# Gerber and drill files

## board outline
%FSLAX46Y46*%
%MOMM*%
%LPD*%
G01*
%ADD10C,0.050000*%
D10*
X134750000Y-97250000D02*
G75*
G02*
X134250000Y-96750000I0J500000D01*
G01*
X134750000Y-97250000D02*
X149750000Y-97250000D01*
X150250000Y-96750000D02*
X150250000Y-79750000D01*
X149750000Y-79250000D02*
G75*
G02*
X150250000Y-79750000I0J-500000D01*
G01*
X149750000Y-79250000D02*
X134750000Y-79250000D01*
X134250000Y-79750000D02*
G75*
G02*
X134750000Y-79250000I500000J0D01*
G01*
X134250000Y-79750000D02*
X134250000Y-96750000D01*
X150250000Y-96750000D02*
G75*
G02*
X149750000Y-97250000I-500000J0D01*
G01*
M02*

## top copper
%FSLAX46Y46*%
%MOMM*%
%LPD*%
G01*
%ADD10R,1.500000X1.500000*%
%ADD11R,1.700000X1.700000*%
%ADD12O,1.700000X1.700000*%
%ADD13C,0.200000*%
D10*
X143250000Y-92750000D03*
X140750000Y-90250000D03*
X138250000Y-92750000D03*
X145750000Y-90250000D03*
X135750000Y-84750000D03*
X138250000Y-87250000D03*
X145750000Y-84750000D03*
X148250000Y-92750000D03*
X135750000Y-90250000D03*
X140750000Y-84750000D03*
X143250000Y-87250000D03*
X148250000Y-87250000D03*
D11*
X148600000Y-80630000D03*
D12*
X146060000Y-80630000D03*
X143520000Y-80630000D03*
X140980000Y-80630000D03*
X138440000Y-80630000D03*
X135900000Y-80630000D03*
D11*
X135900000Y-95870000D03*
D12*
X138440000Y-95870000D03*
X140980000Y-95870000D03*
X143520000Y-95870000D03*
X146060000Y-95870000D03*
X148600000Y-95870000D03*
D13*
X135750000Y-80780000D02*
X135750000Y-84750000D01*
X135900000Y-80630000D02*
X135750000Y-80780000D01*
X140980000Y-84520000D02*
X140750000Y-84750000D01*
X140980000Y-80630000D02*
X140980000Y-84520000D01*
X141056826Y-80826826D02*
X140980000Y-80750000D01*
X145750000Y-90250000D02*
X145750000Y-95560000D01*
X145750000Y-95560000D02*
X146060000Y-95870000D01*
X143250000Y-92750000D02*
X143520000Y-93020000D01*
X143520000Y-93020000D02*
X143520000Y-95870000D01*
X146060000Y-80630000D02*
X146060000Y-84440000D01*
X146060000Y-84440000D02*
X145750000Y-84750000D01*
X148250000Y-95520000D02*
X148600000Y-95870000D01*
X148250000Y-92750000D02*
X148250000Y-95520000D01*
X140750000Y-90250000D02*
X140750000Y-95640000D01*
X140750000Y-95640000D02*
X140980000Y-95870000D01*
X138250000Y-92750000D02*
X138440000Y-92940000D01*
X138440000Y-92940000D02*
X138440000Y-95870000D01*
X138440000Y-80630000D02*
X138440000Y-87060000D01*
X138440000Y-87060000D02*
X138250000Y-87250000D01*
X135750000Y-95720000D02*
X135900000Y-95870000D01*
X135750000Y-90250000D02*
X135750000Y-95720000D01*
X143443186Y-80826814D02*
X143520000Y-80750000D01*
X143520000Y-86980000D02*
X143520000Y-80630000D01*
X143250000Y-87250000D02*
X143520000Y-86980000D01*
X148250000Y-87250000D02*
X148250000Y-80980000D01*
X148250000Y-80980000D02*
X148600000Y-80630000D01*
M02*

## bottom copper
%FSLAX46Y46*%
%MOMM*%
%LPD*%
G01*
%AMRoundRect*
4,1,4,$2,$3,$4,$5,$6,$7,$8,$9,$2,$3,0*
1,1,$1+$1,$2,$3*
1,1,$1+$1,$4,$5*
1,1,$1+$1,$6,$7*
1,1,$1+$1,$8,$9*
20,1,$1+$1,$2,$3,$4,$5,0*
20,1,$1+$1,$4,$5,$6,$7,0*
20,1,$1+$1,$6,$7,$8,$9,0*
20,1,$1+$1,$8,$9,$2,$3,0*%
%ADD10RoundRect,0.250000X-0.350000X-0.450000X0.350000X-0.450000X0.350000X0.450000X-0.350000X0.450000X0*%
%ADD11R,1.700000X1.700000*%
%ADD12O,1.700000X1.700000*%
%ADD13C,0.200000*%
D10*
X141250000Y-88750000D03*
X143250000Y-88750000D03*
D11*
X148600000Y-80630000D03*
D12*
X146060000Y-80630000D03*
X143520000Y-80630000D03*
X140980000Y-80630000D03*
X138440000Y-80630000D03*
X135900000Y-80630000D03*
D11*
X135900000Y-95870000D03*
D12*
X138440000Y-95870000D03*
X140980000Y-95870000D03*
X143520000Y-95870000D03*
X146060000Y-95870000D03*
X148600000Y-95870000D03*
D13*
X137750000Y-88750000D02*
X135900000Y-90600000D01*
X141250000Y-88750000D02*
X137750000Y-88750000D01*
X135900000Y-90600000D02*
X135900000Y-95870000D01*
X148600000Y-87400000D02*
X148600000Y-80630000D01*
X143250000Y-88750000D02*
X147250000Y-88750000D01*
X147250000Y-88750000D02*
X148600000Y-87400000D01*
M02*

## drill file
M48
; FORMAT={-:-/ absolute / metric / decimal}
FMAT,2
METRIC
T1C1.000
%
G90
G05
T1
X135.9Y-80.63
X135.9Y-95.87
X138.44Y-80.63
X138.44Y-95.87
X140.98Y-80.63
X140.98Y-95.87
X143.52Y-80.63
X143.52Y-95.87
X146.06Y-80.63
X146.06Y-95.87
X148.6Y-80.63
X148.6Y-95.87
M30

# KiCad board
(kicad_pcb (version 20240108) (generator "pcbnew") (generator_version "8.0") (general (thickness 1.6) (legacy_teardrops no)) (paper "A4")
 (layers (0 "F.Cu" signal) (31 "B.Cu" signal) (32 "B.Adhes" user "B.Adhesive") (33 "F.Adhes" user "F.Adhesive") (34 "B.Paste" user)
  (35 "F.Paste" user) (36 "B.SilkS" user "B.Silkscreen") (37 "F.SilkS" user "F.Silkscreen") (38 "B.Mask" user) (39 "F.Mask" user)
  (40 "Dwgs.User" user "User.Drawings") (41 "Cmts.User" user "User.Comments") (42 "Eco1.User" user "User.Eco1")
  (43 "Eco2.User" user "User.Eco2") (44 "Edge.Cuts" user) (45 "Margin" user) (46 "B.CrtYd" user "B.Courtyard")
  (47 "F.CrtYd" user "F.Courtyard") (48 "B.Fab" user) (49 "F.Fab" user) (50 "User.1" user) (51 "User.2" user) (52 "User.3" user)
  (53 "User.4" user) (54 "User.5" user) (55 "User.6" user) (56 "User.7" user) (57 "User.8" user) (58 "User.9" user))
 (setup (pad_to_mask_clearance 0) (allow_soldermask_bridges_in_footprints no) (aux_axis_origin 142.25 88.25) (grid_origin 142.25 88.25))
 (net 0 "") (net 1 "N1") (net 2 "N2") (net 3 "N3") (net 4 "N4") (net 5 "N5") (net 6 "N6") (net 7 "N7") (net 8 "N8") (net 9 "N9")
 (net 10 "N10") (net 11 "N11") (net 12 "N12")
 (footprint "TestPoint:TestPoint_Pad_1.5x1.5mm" (layer "F.Cu") (at 143.25 92.75)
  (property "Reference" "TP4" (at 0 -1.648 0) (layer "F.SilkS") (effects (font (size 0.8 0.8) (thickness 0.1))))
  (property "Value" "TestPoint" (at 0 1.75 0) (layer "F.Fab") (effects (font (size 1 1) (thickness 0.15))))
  (pad "1" smd rect (at 0 0) (size 1.5 1.5) (layers "F.Cu" "F.Mask") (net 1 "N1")))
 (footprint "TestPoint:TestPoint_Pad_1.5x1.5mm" (layer "F.Cu") (at 140.75 90.25)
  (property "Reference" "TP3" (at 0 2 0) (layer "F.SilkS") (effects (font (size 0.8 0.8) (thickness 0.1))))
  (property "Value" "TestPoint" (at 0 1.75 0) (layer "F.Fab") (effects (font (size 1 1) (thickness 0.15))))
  (pad "1" smd rect (at 0 0) (size 1.5 1.5) (layers "F.Cu" "F.Mask") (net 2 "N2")))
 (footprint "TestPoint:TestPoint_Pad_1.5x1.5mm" (layer "F.Cu") (at 138.25 92.75)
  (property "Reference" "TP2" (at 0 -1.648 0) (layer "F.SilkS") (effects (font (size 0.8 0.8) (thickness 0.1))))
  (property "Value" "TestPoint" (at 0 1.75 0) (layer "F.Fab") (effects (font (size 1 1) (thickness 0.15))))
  (pad "1" smd rect (at 0 0) (size 1.5 1.5) (layers "F.Cu" "F.Mask") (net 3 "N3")))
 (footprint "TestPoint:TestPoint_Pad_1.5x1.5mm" (layer "F.Cu") (at 145.75 90.25)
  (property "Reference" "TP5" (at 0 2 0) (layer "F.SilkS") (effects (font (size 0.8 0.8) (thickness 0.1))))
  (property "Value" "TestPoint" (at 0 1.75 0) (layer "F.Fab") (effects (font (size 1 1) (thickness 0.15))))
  (pad "1" smd rect (at 0 0) (size 1.5 1.5) (layers "F.Cu" "F.Mask") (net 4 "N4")))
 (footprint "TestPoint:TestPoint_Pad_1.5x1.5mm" (layer "F.Cu") (at 135.75 84.75)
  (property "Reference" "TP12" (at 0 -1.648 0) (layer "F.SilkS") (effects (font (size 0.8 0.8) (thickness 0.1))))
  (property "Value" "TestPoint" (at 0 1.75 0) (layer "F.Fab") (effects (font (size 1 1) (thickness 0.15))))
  (pad "1" smd rect (at 0 0) (size 1.5 1.5) (layers "F.Cu" "F.Mask") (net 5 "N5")))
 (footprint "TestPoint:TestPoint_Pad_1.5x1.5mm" (layer "F.Cu") (at 138.25 87.25)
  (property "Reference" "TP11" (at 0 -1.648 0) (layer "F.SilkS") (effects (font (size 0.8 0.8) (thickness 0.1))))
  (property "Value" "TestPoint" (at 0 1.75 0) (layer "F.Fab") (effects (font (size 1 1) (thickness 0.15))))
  (pad "1" smd rect (at 0 0) (size 1.5 1.5) (layers "F.Cu" "F.Mask") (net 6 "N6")))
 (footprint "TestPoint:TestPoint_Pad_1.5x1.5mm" (layer "F.Cu") (at 145.75 84.75)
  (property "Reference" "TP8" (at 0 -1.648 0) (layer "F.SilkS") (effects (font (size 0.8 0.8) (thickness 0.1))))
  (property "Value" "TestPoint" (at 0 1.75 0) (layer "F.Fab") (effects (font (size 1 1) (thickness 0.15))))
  (pad "1" smd rect (at 0 0) (size 1.5 1.5) (layers "F.Cu" "F.Mask") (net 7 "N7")))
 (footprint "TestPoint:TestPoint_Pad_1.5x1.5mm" (layer "F.Cu") (at 148.25 92.75)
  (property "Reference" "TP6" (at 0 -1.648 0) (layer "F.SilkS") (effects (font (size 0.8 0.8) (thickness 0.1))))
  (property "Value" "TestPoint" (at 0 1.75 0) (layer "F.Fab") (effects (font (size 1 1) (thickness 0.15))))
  (pad "1" smd rect (at 0 0) (size 1.5 1.5) (layers "F.Cu" "F.Mask") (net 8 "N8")))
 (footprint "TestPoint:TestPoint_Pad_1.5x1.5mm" (layer "F.Cu") (at 135.75 90.25)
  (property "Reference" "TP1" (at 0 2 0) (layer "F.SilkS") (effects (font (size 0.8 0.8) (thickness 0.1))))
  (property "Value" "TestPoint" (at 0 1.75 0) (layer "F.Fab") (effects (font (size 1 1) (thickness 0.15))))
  (pad "1" smd rect (at 0 0) (size 1.5 1.5) (layers "F.Cu" "F.Mask") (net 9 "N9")))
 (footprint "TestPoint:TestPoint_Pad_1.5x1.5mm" (layer "F.Cu") (at 140.75 84.75)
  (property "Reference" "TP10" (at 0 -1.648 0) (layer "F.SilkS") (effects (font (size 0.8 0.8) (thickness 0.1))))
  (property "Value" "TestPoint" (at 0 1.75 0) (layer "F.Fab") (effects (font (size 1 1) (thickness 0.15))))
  (pad "1" smd rect (at 0 0) (size 1.5 1.5) (layers "F.Cu" "F.Mask") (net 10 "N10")))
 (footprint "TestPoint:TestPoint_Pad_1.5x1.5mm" (layer "F.Cu") (at 143.25 87.25)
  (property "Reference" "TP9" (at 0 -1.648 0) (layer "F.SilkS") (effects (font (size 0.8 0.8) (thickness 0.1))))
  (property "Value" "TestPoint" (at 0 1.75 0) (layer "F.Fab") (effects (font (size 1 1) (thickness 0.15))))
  (pad "1" smd rect (at 0 0) (size 1.5 1.5) (layers "F.Cu" "F.Mask") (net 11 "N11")))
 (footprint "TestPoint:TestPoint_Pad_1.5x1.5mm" (layer "F.Cu") (at 148.25 87.25)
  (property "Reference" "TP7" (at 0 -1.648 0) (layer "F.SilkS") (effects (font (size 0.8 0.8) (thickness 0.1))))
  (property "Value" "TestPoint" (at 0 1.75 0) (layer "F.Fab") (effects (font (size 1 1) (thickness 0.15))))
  (pad "1" smd rect (at 0 0) (size 1.5 1.5) (layers "F.Cu" "F.Mask") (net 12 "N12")))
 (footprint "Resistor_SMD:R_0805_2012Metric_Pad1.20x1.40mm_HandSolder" (layer "B.Cu") (at 142.25 88.75)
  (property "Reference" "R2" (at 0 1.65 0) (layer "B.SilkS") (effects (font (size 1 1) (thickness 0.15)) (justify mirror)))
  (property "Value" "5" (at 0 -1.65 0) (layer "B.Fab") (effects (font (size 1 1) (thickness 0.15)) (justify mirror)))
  (pad "1" smd roundrect (at -1 0) (size 1.2 1.4) (layers "B.Cu" "B.Paste" "B.Mask") (roundrect_rratio 0.208333) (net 9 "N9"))
  (pad "2" smd roundrect (at 1 0) (size 1.2 1.4) (layers "B.Cu" "B.Paste" "B.Mask") (roundrect_rratio 0.208333) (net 12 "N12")))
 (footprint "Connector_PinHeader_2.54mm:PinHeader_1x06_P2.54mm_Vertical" (layer "B.Cu") (at 148.6 80.63 90)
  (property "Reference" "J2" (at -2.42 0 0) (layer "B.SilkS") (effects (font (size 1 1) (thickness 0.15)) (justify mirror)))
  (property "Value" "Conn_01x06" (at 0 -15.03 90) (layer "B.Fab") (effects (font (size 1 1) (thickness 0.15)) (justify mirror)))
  (pad "1" thru_hole rect (at 0 0 90) (size 1.7 1.7) (drill 1) (layers "*.Cu" "*.Mask") (remove_unused_layers no) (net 12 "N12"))
  (pad "2" thru_hole oval (at 0 -2.54 90) (size 1.7 1.7) (drill 1) (layers "*.Cu" "*.Mask") (remove_unused_layers no) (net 7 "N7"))
  (pad "3" thru_hole oval (at 0 -5.08 90) (size 1.7 1.7) (drill 1) (layers "*.Cu" "*.Mask") (remove_unused_layers no) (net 11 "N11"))
  (pad "4" thru_hole oval (at 0 -7.62 90) (size 1.7 1.7) (drill 1) (layers "*.Cu" "*.Mask") (remove_unused_layers no) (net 10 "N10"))
  (pad "5" thru_hole oval (at 0 -10.16 90) (size 1.7 1.7) (drill 1) (layers "*.Cu" "*.Mask") (remove_unused_layers no) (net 6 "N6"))
  (pad "6" thru_hole oval (at 0 -12.7 90) (size 1.7 1.7) (drill 1) (layers "*.Cu" "*.Mask") (remove_unused_layers no) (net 5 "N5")))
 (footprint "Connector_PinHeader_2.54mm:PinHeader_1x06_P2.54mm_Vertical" (layer "B.Cu") (at 135.9 95.87 -90)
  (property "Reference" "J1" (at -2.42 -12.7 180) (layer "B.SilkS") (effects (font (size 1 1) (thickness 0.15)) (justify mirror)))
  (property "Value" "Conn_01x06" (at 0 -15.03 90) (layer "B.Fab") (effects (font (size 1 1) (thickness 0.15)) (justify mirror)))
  (pad "1" thru_hole rect (at 0 0 270) (size 1.7 1.7) (drill 1) (layers "*.Cu" "*.Mask") (remove_unused_layers no) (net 9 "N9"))
  (pad "2" thru_hole oval (at 0 -2.54 270) (size 1.7 1.7) (drill 1) (layers "*.Cu" "*.Mask") (remove_unused_layers no) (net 3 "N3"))
  (pad "3" thru_hole oval (at 0 -5.08 270) (size 1.7 1.7) (drill 1) (layers "*.Cu" "*.Mask") (remove_unused_layers no) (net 2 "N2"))
  (pad "4" thru_hole oval (at 0 -7.62 270) (size 1.7 1.7) (drill 1) (layers "*.Cu" "*.Mask") (remove_unused_layers no) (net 1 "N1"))
  (pad "5" thru_hole oval (at 0 -10.16 270) (size 1.7 1.7) (drill 1) (layers "*.Cu" "*.Mask") (remove_unused_layers no) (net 4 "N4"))
  (pad "6" thru_hole oval (at 0 -12.7 270) (size 1.7 1.7) (drill 1) (layers "*.Cu" "*.Mask") (remove_unused_layers no) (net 8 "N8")))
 (gr_arc (start 134.75 97.25) (mid 134.396447 97.103553) (end 134.25 96.75) (stroke (width 0.05) (type default)) (layer "Edge.Cuts"))
 (gr_line (start 134.75 97.25) (end 149.75 97.25) (stroke (width 0.05) (type default)) (layer "Edge.Cuts"))
 (gr_line (start 150.25 96.75) (end 150.25 79.75) (stroke (width 0.05) (type default)) (layer "Edge.Cuts"))
 (gr_arc (start 149.75 79.25) (mid 150.103553 79.396447) (end 150.25 79.75) (stroke (width 0.05) (type default)) (layer "Edge.Cuts"))
 (gr_line (start 149.75 79.25) (end 134.75 79.25) (stroke (width 0.05) (type default)) (layer "Edge.Cuts"))
 (gr_arc (start 134.25 79.75) (mid 134.396447 79.396447) (end 134.75 79.25) (stroke (width 0.05) (type default)) (layer "Edge.Cuts"))
 (gr_line (start 134.25 79.75) (end 134.25 96.75) (stroke (width 0.05) (type default)) (layer "Edge.Cuts"))
 (gr_arc (start 150.25 96.75) (mid 150.103553 97.103553) (end 149.75 97.25) (stroke (width 0.05) (type default)) (layer "Edge.Cuts"))
 (segment (start 135.75 80.78) (end 135.75 84.75) (width 0.2) (layer "F.Cu") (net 5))
 (segment (start 135.9 80.63) (end 135.75 80.78) (width 0.2) (layer "F.Cu") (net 5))
 (segment (start 140.98 84.52) (end 140.75 84.75) (width 0.2) (layer "F.Cu") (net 10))
 (segment (start 140.98 80.63) (end 140.98 84.52) (width 0.2) (layer "F.Cu") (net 10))
 (segment (start 141.056826 80.826826) (end 140.98 80.75) (width 0.2) (layer "F.Cu") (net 10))
 (segment (start 145.75 90.25) (end 145.75 95.56) (width 0.2) (layer "F.Cu") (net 4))
 (segment (start 145.75 95.56) (end 146.06 95.87) (width 0.2) (layer "F.Cu") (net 4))
 (segment (start 143.25 92.75) (end 143.52 93.02) (width 0.2) (layer "F.Cu") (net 1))
 (segment (start 143.52 93.02) (end 143.52 95.87) (width 0.2) (layer "F.Cu") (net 1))
 (segment (start 146.06 80.63) (end 146.06 84.44) (width 0.2) (layer "F.Cu") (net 7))
 (segment (start 146.06 84.44) (end 145.75 84.75) (width 0.2) (layer "F.Cu") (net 7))
 (segment (start 148.25 95.52) (end 148.6 95.87) (width 0.2) (layer "F.Cu") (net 8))
 (segment (start 148.25 92.75) (end 148.25 95.52) (width 0.2) (layer "F.Cu") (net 8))
 (segment (start 140.75 90.25) (end 140.75 95.64) (width 0.2) (layer "F.Cu") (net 2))
 (segment (start 140.75 95.64) (end 140.98 95.87) (width 0.2) (layer "F.Cu") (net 2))
 (segment (start 138.25 92.75) (end 138.44 92.94) (width 0.2) (layer "F.Cu") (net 3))
 (segment (start 138.44 92.94) (end 138.44 95.87) (width 0.2) (layer "F.Cu") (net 3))
 (segment (start 138.44 80.63) (end 138.44 87.06) (width 0.2) (layer "F.Cu") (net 6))
 (segment (start 138.44 87.06) (end 138.25 87.25) (width 0.2) (layer "F.Cu") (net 6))
 (segment (start 135.75 95.72) (end 135.9 95.87) (width 0.2) (layer "F.Cu") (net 9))
 (segment (start 135.75 90.25) (end 135.75 95.72) (width 0.2) (layer "F.Cu") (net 9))
 (segment (start 137.75 88.75) (end 135.9 90.6) (width 0.2) (layer "B.Cu") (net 9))
 (segment (start 141.25 88.75) (end 137.75 88.75) (width 0.2) (layer "B.Cu") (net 9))
 (segment (start 135.9 90.6) (end 135.9 95.87) (width 0.2) (layer "B.Cu") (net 9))
 (segment (start 143.443186 80.826814) (end 143.52 80.75) (width 0.2) (layer "F.Cu") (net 11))
 (segment (start 143.52 86.98) (end 143.52 80.63) (width 0.2) (layer "F.Cu") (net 11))
 (segment (start 143.25 87.25) (end 143.52 86.98) (width 0.2) (layer "F.Cu") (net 11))
 (segment (start 148.25 87.25) (end 148.25 80.98) (width 0.2) (layer "F.Cu") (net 12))
 (segment (start 148.25 80.98) (end 148.6 80.63) (width 0.2) (layer "F.Cu") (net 12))
 (segment (start 148.6 87.4) (end 148.6 80.63) (width 0.2) (layer "B.Cu") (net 12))
 (segment (start 143.25 88.75) (end 147.25 88.75) (width 0.2) (layer "B.Cu") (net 12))
 (segment (start 147.25 88.75) (end 148.6 87.4) (width 0.2) (layer "B.Cu") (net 12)))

